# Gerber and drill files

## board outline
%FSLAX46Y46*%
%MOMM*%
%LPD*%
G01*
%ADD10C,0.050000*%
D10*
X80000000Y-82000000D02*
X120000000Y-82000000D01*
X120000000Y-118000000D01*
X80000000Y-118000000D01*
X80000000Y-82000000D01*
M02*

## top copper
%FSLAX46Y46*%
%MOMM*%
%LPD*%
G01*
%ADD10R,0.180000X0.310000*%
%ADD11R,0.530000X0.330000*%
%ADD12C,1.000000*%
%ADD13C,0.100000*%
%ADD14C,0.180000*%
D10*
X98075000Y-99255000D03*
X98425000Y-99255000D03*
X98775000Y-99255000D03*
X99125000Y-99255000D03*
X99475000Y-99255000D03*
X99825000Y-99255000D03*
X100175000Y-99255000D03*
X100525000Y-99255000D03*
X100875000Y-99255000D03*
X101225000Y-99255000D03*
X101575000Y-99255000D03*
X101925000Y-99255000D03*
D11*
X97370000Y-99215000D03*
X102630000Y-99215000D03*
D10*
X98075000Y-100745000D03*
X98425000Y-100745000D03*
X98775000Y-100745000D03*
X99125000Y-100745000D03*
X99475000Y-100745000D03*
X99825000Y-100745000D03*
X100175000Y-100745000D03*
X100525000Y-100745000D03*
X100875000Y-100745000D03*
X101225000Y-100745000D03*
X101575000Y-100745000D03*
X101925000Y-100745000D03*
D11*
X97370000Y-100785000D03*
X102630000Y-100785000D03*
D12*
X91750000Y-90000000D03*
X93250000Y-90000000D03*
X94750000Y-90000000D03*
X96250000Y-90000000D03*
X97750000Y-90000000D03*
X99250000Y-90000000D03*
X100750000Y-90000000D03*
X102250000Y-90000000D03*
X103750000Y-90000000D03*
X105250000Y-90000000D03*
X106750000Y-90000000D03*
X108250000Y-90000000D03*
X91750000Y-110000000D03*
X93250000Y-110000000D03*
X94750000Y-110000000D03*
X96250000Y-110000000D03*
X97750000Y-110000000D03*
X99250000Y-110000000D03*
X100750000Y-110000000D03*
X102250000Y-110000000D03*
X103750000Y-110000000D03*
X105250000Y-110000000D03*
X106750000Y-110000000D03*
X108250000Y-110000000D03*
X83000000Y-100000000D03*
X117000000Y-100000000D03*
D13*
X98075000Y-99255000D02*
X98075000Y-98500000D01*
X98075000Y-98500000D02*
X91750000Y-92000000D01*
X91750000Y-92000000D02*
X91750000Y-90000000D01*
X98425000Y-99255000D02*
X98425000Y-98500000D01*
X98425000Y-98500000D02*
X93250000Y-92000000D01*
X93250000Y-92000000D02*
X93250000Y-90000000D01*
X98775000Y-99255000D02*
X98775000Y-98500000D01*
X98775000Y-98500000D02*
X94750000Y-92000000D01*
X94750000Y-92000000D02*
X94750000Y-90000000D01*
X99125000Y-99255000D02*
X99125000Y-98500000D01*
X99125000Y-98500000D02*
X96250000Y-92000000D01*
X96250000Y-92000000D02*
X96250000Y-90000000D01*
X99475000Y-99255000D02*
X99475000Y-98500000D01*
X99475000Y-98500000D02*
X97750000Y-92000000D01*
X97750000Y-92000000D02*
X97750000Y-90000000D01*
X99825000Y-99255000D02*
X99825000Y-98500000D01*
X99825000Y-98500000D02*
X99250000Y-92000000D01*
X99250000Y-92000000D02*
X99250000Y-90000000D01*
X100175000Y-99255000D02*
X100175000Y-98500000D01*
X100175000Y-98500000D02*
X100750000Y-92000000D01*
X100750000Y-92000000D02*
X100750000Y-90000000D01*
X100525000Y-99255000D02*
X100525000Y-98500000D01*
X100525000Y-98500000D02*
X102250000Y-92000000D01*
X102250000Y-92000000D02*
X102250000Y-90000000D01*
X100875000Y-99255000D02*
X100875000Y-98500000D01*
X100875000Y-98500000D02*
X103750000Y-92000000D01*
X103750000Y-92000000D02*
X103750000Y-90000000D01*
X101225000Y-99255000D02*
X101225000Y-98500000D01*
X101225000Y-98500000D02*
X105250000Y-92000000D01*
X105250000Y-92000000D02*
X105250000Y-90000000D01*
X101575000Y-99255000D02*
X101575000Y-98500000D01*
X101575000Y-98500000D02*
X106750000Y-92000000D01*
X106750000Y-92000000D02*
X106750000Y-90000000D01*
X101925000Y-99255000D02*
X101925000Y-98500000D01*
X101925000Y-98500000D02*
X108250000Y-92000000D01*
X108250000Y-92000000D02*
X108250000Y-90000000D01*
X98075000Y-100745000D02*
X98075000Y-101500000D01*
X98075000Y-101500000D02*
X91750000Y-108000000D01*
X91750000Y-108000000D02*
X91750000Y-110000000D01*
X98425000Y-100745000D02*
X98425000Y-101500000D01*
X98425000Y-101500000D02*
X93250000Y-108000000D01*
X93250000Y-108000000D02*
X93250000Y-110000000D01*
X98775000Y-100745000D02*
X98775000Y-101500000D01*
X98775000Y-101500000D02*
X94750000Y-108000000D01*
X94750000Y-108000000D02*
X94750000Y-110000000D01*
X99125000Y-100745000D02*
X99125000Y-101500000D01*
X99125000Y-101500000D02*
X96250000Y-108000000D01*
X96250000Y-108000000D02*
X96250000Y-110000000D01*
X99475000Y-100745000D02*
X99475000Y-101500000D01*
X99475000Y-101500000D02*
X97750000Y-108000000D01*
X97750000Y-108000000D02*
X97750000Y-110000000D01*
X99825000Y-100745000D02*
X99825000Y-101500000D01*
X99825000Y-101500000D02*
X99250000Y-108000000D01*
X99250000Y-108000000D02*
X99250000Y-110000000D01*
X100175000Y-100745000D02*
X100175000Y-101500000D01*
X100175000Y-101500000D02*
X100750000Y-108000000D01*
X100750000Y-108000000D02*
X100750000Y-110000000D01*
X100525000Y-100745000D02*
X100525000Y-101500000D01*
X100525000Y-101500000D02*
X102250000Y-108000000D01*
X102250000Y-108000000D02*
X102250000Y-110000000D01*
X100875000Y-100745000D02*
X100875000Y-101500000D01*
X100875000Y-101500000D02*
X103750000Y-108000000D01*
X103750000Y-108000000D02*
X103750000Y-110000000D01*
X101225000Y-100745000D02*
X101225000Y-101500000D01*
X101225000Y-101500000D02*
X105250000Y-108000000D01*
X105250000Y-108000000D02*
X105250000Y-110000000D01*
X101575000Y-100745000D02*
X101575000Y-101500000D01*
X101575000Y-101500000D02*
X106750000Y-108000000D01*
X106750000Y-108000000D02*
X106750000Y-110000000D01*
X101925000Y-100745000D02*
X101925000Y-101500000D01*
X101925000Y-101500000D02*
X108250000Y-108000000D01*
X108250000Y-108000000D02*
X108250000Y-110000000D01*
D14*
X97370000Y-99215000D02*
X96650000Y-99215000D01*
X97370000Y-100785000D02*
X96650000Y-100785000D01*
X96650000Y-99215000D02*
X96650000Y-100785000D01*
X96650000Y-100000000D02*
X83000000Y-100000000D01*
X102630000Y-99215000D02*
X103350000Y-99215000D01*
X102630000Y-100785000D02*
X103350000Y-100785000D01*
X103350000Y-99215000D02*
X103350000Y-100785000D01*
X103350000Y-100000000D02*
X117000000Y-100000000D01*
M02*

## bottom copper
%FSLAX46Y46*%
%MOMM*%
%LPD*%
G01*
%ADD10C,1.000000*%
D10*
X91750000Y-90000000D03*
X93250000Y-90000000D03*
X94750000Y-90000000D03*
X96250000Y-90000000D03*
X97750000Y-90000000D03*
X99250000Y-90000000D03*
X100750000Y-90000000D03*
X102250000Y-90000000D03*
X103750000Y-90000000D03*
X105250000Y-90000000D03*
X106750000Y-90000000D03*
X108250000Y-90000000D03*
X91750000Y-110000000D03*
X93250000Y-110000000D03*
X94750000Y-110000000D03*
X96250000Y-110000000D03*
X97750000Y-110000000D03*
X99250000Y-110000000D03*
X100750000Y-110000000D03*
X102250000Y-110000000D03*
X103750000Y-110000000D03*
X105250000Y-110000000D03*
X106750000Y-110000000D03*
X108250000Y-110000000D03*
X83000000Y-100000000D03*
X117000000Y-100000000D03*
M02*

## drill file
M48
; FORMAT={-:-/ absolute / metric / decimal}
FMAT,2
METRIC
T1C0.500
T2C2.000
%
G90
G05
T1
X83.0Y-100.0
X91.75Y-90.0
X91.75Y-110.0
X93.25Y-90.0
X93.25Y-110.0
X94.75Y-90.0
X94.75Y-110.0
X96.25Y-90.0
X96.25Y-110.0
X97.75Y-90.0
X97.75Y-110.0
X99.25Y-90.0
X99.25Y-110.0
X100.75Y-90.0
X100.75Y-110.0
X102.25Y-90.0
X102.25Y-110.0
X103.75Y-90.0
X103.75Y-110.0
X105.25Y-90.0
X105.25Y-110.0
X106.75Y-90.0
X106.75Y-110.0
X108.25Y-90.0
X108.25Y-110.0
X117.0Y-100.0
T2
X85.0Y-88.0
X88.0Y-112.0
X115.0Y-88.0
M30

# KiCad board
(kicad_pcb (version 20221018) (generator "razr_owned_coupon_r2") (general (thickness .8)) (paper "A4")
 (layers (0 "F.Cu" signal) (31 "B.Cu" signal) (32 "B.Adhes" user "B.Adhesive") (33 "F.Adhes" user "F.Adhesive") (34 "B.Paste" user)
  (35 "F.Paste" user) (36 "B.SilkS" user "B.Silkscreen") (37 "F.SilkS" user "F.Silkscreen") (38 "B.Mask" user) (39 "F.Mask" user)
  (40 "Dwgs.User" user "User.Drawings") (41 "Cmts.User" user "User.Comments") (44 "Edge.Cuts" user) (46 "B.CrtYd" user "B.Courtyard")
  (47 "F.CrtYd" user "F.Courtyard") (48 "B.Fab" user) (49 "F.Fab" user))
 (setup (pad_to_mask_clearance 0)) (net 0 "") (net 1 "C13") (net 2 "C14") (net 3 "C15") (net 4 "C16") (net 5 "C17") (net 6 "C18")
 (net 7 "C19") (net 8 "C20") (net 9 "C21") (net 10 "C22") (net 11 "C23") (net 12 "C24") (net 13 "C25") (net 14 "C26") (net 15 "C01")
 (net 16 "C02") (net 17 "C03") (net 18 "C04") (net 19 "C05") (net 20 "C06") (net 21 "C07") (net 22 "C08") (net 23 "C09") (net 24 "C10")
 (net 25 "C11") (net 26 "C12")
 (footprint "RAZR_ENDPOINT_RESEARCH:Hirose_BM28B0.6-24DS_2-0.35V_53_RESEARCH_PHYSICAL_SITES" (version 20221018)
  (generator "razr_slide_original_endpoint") (layer "F.Cu") (at 100 100)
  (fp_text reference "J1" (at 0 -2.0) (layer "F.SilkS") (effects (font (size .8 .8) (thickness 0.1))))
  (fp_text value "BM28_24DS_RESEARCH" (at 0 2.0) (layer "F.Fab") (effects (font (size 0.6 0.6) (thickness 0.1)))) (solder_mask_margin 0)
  (pad "S_NEG_00" smd rect (at -1.925 -0.745) (size 0.18 0.31) (layers "F.Cu" "F.Mask") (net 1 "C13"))
  (pad "S_NEG_01" smd rect (at -1.575 -0.745) (size 0.18 0.31) (layers "F.Cu" "F.Mask") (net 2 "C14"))
  (pad "S_NEG_02" smd rect (at -1.225 -0.745) (size 0.18 0.31) (layers "F.Cu" "F.Mask") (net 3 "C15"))
  (pad "S_NEG_03" smd rect (at -0.875 -0.745) (size 0.18 0.31) (layers "F.Cu" "F.Mask") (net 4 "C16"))
  (pad "S_NEG_04" smd rect (at -0.525 -0.745) (size 0.18 0.31) (layers "F.Cu" "F.Mask") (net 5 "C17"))
  (pad "S_NEG_05" smd rect (at -0.175 -0.745) (size 0.18 0.31) (layers "F.Cu" "F.Mask") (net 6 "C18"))
  (pad "S_NEG_06" smd rect (at 0.175 -0.745) (size 0.18 0.31) (layers "F.Cu" "F.Mask") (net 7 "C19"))
  (pad "S_NEG_07" smd rect (at 0.525 -0.745) (size 0.18 0.31) (layers "F.Cu" "F.Mask") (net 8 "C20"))
  (pad "S_NEG_08" smd rect (at 0.875 -0.745) (size 0.18 0.31) (layers "F.Cu" "F.Mask") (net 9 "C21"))
  (pad "S_NEG_09" smd rect (at 1.225 -0.745) (size 0.18 0.31) (layers "F.Cu" "F.Mask") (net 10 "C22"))
  (pad "S_NEG_10" smd rect (at 1.575 -0.745) (size 0.18 0.31) (layers "F.Cu" "F.Mask") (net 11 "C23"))
  (pad "S_NEG_11" smd rect (at 1.925 -0.745) (size 0.18 0.31) (layers "F.Cu" "F.Mask") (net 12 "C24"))
  (pad "P_L" smd rect (at -2.63 -0.785) (size 0.53 0.33) (layers "F.Cu" "F.Mask") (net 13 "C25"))
  (pad "P_R" smd rect (at 2.63 -0.785) (size 0.53 0.33) (layers "F.Cu" "F.Mask") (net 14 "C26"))
  (pad "S_POS_00" smd rect (at -1.925 0.745) (size 0.18 0.31) (layers "F.Cu" "F.Mask") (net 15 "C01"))
  (pad "S_POS_01" smd rect (at -1.575 0.745) (size 0.18 0.31) (layers "F.Cu" "F.Mask") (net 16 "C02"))
  (pad "S_POS_02" smd rect (at -1.225 0.745) (size 0.18 0.31) (layers "F.Cu" "F.Mask") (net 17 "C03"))
  (pad "S_POS_03" smd rect (at -0.875 0.745) (size 0.18 0.31) (layers "F.Cu" "F.Mask") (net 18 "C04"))
  (pad "S_POS_04" smd rect (at -0.525 0.745) (size 0.18 0.31) (layers "F.Cu" "F.Mask") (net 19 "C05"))
  (pad "S_POS_05" smd rect (at -0.175 0.745) (size 0.18 0.31) (layers "F.Cu" "F.Mask") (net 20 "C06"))
  (pad "S_POS_06" smd rect (at 0.175 0.745) (size 0.18 0.31) (layers "F.Cu" "F.Mask") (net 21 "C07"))
  (pad "S_POS_07" smd rect (at 0.525 0.745) (size 0.18 0.31) (layers "F.Cu" "F.Mask") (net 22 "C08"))
  (pad "S_POS_08" smd rect (at 0.875 0.745) (size 0.18 0.31) (layers "F.Cu" "F.Mask") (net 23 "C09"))
  (pad "S_POS_09" smd rect (at 1.225 0.745) (size 0.18 0.31) (layers "F.Cu" "F.Mask") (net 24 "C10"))
  (pad "S_POS_10" smd rect (at 1.575 0.745) (size 0.18 0.31) (layers "F.Cu" "F.Mask") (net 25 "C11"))
  (pad "S_POS_11" smd rect (at 1.925 0.745) (size 0.18 0.31) (layers "F.Cu" "F.Mask") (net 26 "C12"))
  (pad "P_L" smd rect (at -2.63 0.785) (size 0.53 0.33) (layers "F.Cu" "F.Mask") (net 13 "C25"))
  (pad "P_R" smd rect (at 2.63 0.785) (size 0.53 0.33) (layers "F.Cu" "F.Mask") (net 14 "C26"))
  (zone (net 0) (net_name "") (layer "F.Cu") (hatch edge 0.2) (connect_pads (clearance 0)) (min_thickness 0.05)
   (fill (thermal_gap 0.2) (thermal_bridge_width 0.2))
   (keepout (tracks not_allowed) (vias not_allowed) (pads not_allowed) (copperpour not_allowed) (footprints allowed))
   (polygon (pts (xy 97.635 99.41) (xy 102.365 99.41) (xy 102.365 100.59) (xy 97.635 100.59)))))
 (segment (start 98.075000 99.255000) (end 98.075000 98.500000) (width 0.1) (layer "F.Cu") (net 1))
 (segment (start 98.075000 98.500000) (end 91.750000 92.000000) (width 0.1) (layer "F.Cu") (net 1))
 (segment (start 91.750000 92.000000) (end 91.750000 90.000000) (width 0.1) (layer "F.Cu") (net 1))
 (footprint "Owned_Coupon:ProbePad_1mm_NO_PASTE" (layer "F.Cu") (at 91.75 90)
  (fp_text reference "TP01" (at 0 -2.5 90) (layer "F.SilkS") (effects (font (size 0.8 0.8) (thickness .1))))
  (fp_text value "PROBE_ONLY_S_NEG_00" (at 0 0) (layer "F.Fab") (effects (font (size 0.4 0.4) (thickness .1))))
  (pad "1" thru_hole circle (at 0 0) (size 1 1) (drill .5) (layers "*.Cu" "*.Mask") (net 1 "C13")))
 (segment (start 98.425000 99.255000) (end 98.425000 98.500000) (width 0.1) (layer "F.Cu") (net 2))
 (segment (start 98.425000 98.500000) (end 93.250000 92.000000) (width 0.1) (layer "F.Cu") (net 2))
 (segment (start 93.250000 92.000000) (end 93.250000 90.000000) (width 0.1) (layer "F.Cu") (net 2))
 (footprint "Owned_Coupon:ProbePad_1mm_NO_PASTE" (layer "F.Cu") (at 93.25 90)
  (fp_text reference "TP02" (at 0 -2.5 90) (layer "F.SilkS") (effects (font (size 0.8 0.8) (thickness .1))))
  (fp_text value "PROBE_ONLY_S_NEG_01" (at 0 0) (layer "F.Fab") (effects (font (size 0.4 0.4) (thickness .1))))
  (pad "1" thru_hole circle (at 0 0) (size 1 1) (drill .5) (layers "*.Cu" "*.Mask") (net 2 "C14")))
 (segment (start 98.775000 99.255000) (end 98.775000 98.500000) (width 0.1) (layer "F.Cu") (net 3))
 (segment (start 98.775000 98.500000) (end 94.750000 92.000000) (width 0.1) (layer "F.Cu") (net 3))
 (segment (start 94.750000 92.000000) (end 94.750000 90.000000) (width 0.1) (layer "F.Cu") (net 3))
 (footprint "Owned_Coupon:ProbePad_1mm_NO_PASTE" (layer "F.Cu") (at 94.75 90)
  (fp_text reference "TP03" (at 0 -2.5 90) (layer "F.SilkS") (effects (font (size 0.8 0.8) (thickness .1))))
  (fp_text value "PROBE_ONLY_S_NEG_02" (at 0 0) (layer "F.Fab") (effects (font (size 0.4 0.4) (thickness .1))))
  (pad "1" thru_hole circle (at 0 0) (size 1 1) (drill .5) (layers "*.Cu" "*.Mask") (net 3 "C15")))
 (segment (start 99.125000 99.255000) (end 99.125000 98.500000) (width 0.1) (layer "F.Cu") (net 4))
 (segment (start 99.125000 98.500000) (end 96.250000 92.000000) (width 0.1) (layer "F.Cu") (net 4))
 (segment (start 96.250000 92.000000) (end 96.250000 90.000000) (width 0.1) (layer "F.Cu") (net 4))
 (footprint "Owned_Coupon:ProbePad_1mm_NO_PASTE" (layer "F.Cu") (at 96.25 90)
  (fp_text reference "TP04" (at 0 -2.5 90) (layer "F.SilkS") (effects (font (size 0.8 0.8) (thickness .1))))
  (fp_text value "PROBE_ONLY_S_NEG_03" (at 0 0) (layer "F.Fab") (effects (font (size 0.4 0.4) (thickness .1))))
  (pad "1" thru_hole circle (at 0 0) (size 1 1) (drill .5) (layers "*.Cu" "*.Mask") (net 4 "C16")))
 (segment (start 99.475000 99.255000) (end 99.475000 98.500000) (width 0.1) (layer "F.Cu") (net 5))
 (segment (start 99.475000 98.500000) (end 97.750000 92.000000) (width 0.1) (layer "F.Cu") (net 5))
 (segment (start 97.750000 92.000000) (end 97.750000 90.000000) (width 0.1) (layer "F.Cu") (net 5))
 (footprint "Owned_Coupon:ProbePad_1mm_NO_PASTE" (layer "F.Cu") (at 97.75 90)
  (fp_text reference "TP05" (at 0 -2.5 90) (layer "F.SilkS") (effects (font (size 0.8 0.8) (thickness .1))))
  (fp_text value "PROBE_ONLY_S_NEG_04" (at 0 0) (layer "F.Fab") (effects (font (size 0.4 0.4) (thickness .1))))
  (pad "1" thru_hole circle (at 0 0) (size 1 1) (drill .5) (layers "*.Cu" "*.Mask") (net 5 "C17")))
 (segment (start 99.825000 99.255000) (end 99.825000 98.500000) (width 0.1) (layer "F.Cu") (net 6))
 (segment (start 99.825000 98.500000) (end 99.250000 92.000000) (width 0.1) (layer "F.Cu") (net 6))
 (segment (start 99.250000 92.000000) (end 99.250000 90.000000) (width 0.1) (layer "F.Cu") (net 6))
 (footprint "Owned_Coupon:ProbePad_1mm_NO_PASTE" (layer "F.Cu") (at 99.25 90)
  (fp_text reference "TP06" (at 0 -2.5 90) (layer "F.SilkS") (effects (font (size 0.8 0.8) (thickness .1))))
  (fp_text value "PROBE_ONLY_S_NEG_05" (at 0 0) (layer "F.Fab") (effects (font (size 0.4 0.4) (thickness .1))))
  (pad "1" thru_hole circle (at 0 0) (size 1 1) (drill .5) (layers "*.Cu" "*.Mask") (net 6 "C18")))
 (segment (start 100.175000 99.255000) (end 100.175000 98.500000) (width 0.1) (layer "F.Cu") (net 7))
 (segment (start 100.175000 98.500000) (end 100.750000 92.000000) (width 0.1) (layer "F.Cu") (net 7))
 (segment (start 100.750000 92.000000) (end 100.750000 90.000000) (width 0.1) (layer "F.Cu") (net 7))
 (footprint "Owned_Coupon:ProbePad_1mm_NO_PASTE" (layer "F.Cu") (at 100.75 90)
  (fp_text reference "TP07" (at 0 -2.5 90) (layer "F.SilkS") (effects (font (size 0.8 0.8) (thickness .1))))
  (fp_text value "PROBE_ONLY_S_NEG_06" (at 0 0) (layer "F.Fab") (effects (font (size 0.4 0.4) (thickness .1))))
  (pad "1" thru_hole circle (at 0 0) (size 1 1) (drill .5) (layers "*.Cu" "*.Mask") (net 7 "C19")))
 (segment (start 100.525000 99.255000) (end 100.525000 98.500000) (width 0.1) (layer "F.Cu") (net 8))
 (segment (start 100.525000 98.500000) (end 102.250000 92.000000) (width 0.1) (layer "F.Cu") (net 8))
 (segment (start 102.250000 92.000000) (end 102.250000 90.000000) (width 0.1) (layer "F.Cu") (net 8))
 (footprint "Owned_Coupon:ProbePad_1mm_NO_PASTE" (layer "F.Cu") (at 102.25 90)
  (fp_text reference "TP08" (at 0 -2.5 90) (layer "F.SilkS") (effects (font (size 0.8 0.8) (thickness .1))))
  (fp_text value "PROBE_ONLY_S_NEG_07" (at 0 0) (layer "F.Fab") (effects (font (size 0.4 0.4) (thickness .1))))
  (pad "1" thru_hole circle (at 0 0) (size 1 1) (drill .5) (layers "*.Cu" "*.Mask") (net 8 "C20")))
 (segment (start 100.875000 99.255000) (end 100.875000 98.500000) (width 0.1) (layer "F.Cu") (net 9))
 (segment (start 100.875000 98.500000) (end 103.750000 92.000000) (width 0.1) (layer "F.Cu") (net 9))
 (segment (start 103.750000 92.000000) (end 103.750000 90.000000) (width 0.1) (layer "F.Cu") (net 9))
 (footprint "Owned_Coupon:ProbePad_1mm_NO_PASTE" (layer "F.Cu") (at 103.75 90)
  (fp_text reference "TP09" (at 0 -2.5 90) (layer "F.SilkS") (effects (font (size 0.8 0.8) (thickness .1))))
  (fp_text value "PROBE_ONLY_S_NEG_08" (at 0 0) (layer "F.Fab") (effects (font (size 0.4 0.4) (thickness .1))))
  (pad "1" thru_hole circle (at 0 0) (size 1 1) (drill .5) (layers "*.Cu" "*.Mask") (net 9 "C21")))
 (segment (start 101.225000 99.255000) (end 101.225000 98.500000) (width 0.1) (layer "F.Cu") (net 10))
 (segment (start 101.225000 98.500000) (end 105.250000 92.000000) (width 0.1) (layer "F.Cu") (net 10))
 (segment (start 105.250000 92.000000) (end 105.250000 90.000000) (width 0.1) (layer "F.Cu") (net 10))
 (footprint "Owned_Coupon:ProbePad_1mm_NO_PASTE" (layer "F.Cu") (at 105.25 90)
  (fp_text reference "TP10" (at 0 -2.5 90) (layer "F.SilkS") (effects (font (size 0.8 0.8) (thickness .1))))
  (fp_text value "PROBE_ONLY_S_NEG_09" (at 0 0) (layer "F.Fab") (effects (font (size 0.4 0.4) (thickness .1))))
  (pad "1" thru_hole circle (at 0 0) (size 1 1) (drill .5) (layers "*.Cu" "*.Mask") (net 10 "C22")))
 (segment (start 101.575000 99.255000) (end 101.575000 98.500000) (width 0.1) (layer "F.Cu") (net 11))
 (segment (start 101.575000 98.500000) (end 106.750000 92.000000) (width 0.1) (layer "F.Cu") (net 11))
 (segment (start 106.750000 92.000000) (end 106.750000 90.000000) (width 0.1) (layer "F.Cu") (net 11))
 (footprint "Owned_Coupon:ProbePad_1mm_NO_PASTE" (layer "F.Cu") (at 106.75 90)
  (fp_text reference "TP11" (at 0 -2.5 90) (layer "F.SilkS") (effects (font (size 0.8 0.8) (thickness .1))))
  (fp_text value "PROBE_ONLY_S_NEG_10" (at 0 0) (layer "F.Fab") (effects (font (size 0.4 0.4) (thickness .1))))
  (pad "1" thru_hole circle (at 0 0) (size 1 1) (drill .5) (layers "*.Cu" "*.Mask") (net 11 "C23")))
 (segment (start 101.925000 99.255000) (end 101.925000 98.500000) (width 0.1) (layer "F.Cu") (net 12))
 (segment (start 101.925000 98.500000) (end 108.250000 92.000000) (width 0.1) (layer "F.Cu") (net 12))
 (segment (start 108.250000 92.000000) (end 108.250000 90.000000) (width 0.1) (layer "F.Cu") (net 12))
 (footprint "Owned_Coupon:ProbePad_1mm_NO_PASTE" (layer "F.Cu") (at 108.25 90)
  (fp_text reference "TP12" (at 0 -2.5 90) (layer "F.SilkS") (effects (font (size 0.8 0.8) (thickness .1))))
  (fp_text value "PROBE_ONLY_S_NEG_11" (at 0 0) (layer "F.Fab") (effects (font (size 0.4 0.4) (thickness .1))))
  (pad "1" thru_hole circle (at 0 0) (size 1 1) (drill .5) (layers "*.Cu" "*.Mask") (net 12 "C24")))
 (segment (start 98.075000 100.745000) (end 98.075000 101.500000) (width 0.1) (layer "F.Cu") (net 15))
 (segment (start 98.075000 101.500000) (end 91.750000 108.000000) (width 0.1) (layer "F.Cu") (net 15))
 (segment (start 91.750000 108.000000) (end 91.750000 110.000000) (width 0.1) (layer "F.Cu") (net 15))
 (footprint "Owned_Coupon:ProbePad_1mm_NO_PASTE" (layer "F.Cu") (at 91.75 110)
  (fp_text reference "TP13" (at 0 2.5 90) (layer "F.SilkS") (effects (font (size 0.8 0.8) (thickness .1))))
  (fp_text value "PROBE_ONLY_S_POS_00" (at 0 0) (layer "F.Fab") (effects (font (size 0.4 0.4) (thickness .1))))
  (pad "1" thru_hole circle (at 0 0) (size 1 1) (drill .5) (layers "*.Cu" "*.Mask") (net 15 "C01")))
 (segment (start 98.425000 100.745000) (end 98.425000 101.500000) (width 0.1) (layer "F.Cu") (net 16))
 (segment (start 98.425000 101.500000) (end 93.250000 108.000000) (width 0.1) (layer "F.Cu") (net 16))
 (segment (start 93.250000 108.000000) (end 93.250000 110.000000) (width 0.1) (layer "F.Cu") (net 16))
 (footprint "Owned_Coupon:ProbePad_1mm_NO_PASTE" (layer "F.Cu") (at 93.25 110)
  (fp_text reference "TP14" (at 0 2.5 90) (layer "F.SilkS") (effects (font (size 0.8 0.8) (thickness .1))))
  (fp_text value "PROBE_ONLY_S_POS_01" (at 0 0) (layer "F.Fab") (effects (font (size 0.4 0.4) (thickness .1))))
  (pad "1" thru_hole circle (at 0 0) (size 1 1) (drill .5) (layers "*.Cu" "*.Mask") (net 16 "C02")))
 (segment (start 98.775000 100.745000) (end 98.775000 101.500000) (width 0.1) (layer "F.Cu") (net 17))
 (segment (start 98.775000 101.500000) (end 94.750000 108.000000) (width 0.1) (layer "F.Cu") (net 17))
 (segment (start 94.750000 108.000000) (end 94.750000 110.000000) (width 0.1) (layer "F.Cu") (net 17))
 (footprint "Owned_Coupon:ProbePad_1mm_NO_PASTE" (layer "F.Cu") (at 94.75 110)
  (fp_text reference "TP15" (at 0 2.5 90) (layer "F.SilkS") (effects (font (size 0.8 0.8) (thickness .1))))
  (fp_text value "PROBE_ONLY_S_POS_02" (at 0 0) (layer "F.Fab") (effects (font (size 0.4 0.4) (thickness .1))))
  (pad "1" thru_hole circle (at 0 0) (size 1 1) (drill .5) (layers "*.Cu" "*.Mask") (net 17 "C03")))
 (segment (start 99.125000 100.745000) (end 99.125000 101.500000) (width 0.1) (layer "F.Cu") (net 18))
 (segment (start 99.125000 101.500000) (end 96.250000 108.000000) (width 0.1) (layer "F.Cu") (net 18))
 (segment (start 96.250000 108.000000) (end 96.250000 110.000000) (width 0.1) (layer "F.Cu") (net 18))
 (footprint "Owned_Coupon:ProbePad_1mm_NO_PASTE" (layer "F.Cu") (at 96.25 110)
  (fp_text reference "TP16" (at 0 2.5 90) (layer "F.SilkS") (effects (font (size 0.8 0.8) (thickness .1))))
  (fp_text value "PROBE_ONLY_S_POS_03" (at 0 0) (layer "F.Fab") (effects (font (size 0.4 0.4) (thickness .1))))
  (pad "1" thru_hole circle (at 0 0) (size 1 1) (drill .5) (layers "*.Cu" "*.Mask") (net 18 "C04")))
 (segment (start 99.475000 100.745000) (end 99.475000 101.500000) (width 0.1) (layer "F.Cu") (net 19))
 (segment (start 99.475000 101.500000) (end 97.750000 108.000000) (width 0.1) (layer "F.Cu") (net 19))
 (segment (start 97.750000 108.000000) (end 97.750000 110.000000) (width 0.1) (layer "F.Cu") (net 19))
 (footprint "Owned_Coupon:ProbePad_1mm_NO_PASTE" (layer "F.Cu") (at 97.75 110)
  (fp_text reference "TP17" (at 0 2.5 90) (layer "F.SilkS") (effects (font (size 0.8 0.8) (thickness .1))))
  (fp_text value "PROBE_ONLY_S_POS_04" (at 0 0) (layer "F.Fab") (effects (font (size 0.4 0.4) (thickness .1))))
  (pad "1" thru_hole circle (at 0 0) (size 1 1) (drill .5) (layers "*.Cu" "*.Mask") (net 19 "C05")))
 (segment (start 99.825000 100.745000) (end 99.825000 101.500000) (width 0.1) (layer "F.Cu") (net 20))
 (segment (start 99.825000 101.500000) (end 99.250000 108.000000) (width 0.1) (layer "F.Cu") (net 20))
 (segment (start 99.250000 108.000000) (end 99.250000 110.000000) (width 0.1) (layer "F.Cu") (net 20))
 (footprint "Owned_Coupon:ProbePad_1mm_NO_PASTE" (layer "F.Cu") (at 99.25 110)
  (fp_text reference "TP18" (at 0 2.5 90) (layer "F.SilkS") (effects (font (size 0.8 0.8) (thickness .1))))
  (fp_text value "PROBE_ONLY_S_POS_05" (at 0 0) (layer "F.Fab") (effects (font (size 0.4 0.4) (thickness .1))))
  (pad "1" thru_hole circle (at 0 0) (size 1 1) (drill .5) (layers "*.Cu" "*.Mask") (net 20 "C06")))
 (segment (start 100.175000 100.745000) (end 100.175000 101.500000) (width 0.1) (layer "F.Cu") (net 21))
 (segment (start 100.175000 101.500000) (end 100.750000 108.000000) (width 0.1) (layer "F.Cu") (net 21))
 (segment (start 100.750000 108.000000) (end 100.750000 110.000000) (width 0.1) (layer "F.Cu") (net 21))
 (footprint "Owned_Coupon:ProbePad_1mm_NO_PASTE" (layer "F.Cu") (at 100.75 110)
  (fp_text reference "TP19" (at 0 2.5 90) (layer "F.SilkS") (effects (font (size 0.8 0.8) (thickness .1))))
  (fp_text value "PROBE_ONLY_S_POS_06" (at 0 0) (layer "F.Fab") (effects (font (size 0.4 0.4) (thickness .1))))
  (pad "1" thru_hole circle (at 0 0) (size 1 1) (drill .5) (layers "*.Cu" "*.Mask") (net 21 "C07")))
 (segment (start 100.525000 100.745000) (end 100.525000 101.500000) (width 0.1) (layer "F.Cu") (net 22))
 (segment (start 100.525000 101.500000) (end 102.250000 108.000000) (width 0.1) (layer "F.Cu") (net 22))
 (segment (start 102.250000 108.000000) (end 102.250000 110.000000) (width 0.1) (layer "F.Cu") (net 22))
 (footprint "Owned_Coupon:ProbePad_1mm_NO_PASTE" (layer "F.Cu") (at 102.25 110)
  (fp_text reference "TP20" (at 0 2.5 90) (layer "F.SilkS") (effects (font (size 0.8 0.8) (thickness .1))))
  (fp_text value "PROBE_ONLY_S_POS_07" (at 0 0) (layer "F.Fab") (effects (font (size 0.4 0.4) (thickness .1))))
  (pad "1" thru_hole circle (at 0 0) (size 1 1) (drill .5) (layers "*.Cu" "*.Mask") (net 22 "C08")))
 (segment (start 100.875000 100.745000) (end 100.875000 101.500000) (width 0.1) (layer "F.Cu") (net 23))
 (segment (start 100.875000 101.500000) (end 103.750000 108.000000) (width 0.1) (layer "F.Cu") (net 23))
 (segment (start 103.750000 108.000000) (end 103.750000 110.000000) (width 0.1) (layer "F.Cu") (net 23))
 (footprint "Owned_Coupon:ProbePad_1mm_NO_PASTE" (layer "F.Cu") (at 103.75 110)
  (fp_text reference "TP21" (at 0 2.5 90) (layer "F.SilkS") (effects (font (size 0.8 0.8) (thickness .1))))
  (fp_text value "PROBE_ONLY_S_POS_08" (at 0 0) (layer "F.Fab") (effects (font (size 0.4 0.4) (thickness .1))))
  (pad "1" thru_hole circle (at 0 0) (size 1 1) (drill .5) (layers "*.Cu" "*.Mask") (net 23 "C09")))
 (segment (start 101.225000 100.745000) (end 101.225000 101.500000) (width 0.1) (layer "F.Cu") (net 24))
 (segment (start 101.225000 101.500000) (end 105.250000 108.000000) (width 0.1) (layer "F.Cu") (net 24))
 (segment (start 105.250000 108.000000) (end 105.250000 110.000000) (width 0.1) (layer "F.Cu") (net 24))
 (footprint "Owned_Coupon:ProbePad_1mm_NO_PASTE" (layer "F.Cu") (at 105.25 110)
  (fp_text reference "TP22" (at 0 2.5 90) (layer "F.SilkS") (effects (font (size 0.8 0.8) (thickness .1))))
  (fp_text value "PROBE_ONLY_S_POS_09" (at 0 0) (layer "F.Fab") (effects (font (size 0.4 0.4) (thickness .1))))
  (pad "1" thru_hole circle (at 0 0) (size 1 1) (drill .5) (layers "*.Cu" "*.Mask") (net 24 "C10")))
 (segment (start 101.575000 100.745000) (end 101.575000 101.500000) (width 0.1) (layer "F.Cu") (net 25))
 (segment (start 101.575000 101.500000) (end 106.750000 108.000000) (width 0.1) (layer "F.Cu") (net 25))
 (segment (start 106.750000 108.000000) (end 106.750000 110.000000) (width 0.1) (layer "F.Cu") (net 25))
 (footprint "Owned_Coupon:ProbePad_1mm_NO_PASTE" (layer "F.Cu") (at 106.75 110)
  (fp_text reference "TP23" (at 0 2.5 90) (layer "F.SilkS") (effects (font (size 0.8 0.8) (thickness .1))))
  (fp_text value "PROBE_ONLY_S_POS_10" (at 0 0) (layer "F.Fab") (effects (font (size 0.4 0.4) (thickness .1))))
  (pad "1" thru_hole circle (at 0 0) (size 1 1) (drill .5) (layers "*.Cu" "*.Mask") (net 25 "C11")))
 (segment (start 101.925000 100.745000) (end 101.925000 101.500000) (width 0.1) (layer "F.Cu") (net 26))
 (segment (start 101.925000 101.500000) (end 108.250000 108.000000) (width 0.1) (layer "F.Cu") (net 26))
 (segment (start 108.250000 108.000000) (end 108.250000 110.000000) (width 0.1) (layer "F.Cu") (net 26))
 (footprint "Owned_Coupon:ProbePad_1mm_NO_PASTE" (layer "F.Cu") (at 108.25 110)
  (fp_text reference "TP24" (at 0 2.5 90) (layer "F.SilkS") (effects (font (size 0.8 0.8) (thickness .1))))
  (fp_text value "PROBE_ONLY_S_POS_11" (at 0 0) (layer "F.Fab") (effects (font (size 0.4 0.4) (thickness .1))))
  (pad "1" thru_hole circle (at 0 0) (size 1 1) (drill .5) (layers "*.Cu" "*.Mask") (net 26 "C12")))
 (segment (start 97.370000 99.215000) (end 96.650000 99.215000) (width 0.18) (layer "F.Cu") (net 13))
 (segment (start 97.370000 100.785000) (end 96.650000 100.785000) (width 0.18) (layer "F.Cu") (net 13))
 (segment (start 96.650000 99.215000) (end 96.650000 100.785000) (width 0.18) (layer "F.Cu") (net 13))
 (segment (start 96.650000 100.000000) (end 83.000000 100.000000) (width 0.18) (layer "F.Cu") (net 13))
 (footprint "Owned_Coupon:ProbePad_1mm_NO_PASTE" (layer "F.Cu") (at 83 100)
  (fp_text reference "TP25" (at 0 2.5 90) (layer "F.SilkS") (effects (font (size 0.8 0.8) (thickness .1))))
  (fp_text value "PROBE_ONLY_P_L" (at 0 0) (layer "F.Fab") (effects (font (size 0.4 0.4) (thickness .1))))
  (pad "1" thru_hole circle (at 0 0) (size 1 1) (drill .5) (layers "*.Cu" "*.Mask") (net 13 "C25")))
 (segment (start 102.630000 99.215000) (end 103.350000 99.215000) (width 0.18) (layer "F.Cu") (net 14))
 (segment (start 102.630000 100.785000) (end 103.350000 100.785000) (width 0.18) (layer "F.Cu") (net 14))
 (segment (start 103.350000 99.215000) (end 103.350000 100.785000) (width 0.18) (layer "F.Cu") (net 14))
 (segment (start 103.350000 100.000000) (end 117.000000 100.000000) (width 0.18) (layer "F.Cu") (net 14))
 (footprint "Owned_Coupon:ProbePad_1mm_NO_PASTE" (layer "F.Cu") (at 117 100)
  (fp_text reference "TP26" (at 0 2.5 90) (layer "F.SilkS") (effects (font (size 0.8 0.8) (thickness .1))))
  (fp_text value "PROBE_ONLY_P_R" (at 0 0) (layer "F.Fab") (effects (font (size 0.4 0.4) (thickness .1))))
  (pad "1" thru_hole circle (at 0 0) (size 1 1) (drill .5) (layers "*.Cu" "*.Mask") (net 14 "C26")))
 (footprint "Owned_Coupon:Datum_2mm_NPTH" (layer "F.Cu") (at 85 88)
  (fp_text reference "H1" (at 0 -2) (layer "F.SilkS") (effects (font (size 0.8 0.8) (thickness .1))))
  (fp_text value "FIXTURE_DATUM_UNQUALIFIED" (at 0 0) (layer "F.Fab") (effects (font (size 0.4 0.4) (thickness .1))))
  (pad "" np_thru_hole circle (at 0 0) (size 2 2) (drill 2) (layers "*.Cu" "*.Mask")))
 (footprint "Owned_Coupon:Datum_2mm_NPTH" (layer "F.Cu") (at 115 88)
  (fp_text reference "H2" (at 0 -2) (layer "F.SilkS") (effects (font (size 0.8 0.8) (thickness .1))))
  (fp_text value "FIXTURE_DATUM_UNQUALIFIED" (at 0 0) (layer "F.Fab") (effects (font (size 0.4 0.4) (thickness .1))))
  (pad "" np_thru_hole circle (at 0 0) (size 2 2) (drill 2) (layers "*.Cu" "*.Mask")))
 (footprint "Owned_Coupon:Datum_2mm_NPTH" (layer "F.Cu") (at 88 112)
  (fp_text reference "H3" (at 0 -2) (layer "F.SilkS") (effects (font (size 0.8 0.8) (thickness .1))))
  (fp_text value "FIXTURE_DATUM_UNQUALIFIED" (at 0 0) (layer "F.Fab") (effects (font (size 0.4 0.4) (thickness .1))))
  (pad "" np_thru_hole circle (at 0 0) (size 2 2) (drill 2) (layers "*.Cu" "*.Mask")))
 (gr_rect (start 80 82) (end 120 118) (stroke (width .05) (type default)) (fill none) (layer "Edge.Cuts")))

